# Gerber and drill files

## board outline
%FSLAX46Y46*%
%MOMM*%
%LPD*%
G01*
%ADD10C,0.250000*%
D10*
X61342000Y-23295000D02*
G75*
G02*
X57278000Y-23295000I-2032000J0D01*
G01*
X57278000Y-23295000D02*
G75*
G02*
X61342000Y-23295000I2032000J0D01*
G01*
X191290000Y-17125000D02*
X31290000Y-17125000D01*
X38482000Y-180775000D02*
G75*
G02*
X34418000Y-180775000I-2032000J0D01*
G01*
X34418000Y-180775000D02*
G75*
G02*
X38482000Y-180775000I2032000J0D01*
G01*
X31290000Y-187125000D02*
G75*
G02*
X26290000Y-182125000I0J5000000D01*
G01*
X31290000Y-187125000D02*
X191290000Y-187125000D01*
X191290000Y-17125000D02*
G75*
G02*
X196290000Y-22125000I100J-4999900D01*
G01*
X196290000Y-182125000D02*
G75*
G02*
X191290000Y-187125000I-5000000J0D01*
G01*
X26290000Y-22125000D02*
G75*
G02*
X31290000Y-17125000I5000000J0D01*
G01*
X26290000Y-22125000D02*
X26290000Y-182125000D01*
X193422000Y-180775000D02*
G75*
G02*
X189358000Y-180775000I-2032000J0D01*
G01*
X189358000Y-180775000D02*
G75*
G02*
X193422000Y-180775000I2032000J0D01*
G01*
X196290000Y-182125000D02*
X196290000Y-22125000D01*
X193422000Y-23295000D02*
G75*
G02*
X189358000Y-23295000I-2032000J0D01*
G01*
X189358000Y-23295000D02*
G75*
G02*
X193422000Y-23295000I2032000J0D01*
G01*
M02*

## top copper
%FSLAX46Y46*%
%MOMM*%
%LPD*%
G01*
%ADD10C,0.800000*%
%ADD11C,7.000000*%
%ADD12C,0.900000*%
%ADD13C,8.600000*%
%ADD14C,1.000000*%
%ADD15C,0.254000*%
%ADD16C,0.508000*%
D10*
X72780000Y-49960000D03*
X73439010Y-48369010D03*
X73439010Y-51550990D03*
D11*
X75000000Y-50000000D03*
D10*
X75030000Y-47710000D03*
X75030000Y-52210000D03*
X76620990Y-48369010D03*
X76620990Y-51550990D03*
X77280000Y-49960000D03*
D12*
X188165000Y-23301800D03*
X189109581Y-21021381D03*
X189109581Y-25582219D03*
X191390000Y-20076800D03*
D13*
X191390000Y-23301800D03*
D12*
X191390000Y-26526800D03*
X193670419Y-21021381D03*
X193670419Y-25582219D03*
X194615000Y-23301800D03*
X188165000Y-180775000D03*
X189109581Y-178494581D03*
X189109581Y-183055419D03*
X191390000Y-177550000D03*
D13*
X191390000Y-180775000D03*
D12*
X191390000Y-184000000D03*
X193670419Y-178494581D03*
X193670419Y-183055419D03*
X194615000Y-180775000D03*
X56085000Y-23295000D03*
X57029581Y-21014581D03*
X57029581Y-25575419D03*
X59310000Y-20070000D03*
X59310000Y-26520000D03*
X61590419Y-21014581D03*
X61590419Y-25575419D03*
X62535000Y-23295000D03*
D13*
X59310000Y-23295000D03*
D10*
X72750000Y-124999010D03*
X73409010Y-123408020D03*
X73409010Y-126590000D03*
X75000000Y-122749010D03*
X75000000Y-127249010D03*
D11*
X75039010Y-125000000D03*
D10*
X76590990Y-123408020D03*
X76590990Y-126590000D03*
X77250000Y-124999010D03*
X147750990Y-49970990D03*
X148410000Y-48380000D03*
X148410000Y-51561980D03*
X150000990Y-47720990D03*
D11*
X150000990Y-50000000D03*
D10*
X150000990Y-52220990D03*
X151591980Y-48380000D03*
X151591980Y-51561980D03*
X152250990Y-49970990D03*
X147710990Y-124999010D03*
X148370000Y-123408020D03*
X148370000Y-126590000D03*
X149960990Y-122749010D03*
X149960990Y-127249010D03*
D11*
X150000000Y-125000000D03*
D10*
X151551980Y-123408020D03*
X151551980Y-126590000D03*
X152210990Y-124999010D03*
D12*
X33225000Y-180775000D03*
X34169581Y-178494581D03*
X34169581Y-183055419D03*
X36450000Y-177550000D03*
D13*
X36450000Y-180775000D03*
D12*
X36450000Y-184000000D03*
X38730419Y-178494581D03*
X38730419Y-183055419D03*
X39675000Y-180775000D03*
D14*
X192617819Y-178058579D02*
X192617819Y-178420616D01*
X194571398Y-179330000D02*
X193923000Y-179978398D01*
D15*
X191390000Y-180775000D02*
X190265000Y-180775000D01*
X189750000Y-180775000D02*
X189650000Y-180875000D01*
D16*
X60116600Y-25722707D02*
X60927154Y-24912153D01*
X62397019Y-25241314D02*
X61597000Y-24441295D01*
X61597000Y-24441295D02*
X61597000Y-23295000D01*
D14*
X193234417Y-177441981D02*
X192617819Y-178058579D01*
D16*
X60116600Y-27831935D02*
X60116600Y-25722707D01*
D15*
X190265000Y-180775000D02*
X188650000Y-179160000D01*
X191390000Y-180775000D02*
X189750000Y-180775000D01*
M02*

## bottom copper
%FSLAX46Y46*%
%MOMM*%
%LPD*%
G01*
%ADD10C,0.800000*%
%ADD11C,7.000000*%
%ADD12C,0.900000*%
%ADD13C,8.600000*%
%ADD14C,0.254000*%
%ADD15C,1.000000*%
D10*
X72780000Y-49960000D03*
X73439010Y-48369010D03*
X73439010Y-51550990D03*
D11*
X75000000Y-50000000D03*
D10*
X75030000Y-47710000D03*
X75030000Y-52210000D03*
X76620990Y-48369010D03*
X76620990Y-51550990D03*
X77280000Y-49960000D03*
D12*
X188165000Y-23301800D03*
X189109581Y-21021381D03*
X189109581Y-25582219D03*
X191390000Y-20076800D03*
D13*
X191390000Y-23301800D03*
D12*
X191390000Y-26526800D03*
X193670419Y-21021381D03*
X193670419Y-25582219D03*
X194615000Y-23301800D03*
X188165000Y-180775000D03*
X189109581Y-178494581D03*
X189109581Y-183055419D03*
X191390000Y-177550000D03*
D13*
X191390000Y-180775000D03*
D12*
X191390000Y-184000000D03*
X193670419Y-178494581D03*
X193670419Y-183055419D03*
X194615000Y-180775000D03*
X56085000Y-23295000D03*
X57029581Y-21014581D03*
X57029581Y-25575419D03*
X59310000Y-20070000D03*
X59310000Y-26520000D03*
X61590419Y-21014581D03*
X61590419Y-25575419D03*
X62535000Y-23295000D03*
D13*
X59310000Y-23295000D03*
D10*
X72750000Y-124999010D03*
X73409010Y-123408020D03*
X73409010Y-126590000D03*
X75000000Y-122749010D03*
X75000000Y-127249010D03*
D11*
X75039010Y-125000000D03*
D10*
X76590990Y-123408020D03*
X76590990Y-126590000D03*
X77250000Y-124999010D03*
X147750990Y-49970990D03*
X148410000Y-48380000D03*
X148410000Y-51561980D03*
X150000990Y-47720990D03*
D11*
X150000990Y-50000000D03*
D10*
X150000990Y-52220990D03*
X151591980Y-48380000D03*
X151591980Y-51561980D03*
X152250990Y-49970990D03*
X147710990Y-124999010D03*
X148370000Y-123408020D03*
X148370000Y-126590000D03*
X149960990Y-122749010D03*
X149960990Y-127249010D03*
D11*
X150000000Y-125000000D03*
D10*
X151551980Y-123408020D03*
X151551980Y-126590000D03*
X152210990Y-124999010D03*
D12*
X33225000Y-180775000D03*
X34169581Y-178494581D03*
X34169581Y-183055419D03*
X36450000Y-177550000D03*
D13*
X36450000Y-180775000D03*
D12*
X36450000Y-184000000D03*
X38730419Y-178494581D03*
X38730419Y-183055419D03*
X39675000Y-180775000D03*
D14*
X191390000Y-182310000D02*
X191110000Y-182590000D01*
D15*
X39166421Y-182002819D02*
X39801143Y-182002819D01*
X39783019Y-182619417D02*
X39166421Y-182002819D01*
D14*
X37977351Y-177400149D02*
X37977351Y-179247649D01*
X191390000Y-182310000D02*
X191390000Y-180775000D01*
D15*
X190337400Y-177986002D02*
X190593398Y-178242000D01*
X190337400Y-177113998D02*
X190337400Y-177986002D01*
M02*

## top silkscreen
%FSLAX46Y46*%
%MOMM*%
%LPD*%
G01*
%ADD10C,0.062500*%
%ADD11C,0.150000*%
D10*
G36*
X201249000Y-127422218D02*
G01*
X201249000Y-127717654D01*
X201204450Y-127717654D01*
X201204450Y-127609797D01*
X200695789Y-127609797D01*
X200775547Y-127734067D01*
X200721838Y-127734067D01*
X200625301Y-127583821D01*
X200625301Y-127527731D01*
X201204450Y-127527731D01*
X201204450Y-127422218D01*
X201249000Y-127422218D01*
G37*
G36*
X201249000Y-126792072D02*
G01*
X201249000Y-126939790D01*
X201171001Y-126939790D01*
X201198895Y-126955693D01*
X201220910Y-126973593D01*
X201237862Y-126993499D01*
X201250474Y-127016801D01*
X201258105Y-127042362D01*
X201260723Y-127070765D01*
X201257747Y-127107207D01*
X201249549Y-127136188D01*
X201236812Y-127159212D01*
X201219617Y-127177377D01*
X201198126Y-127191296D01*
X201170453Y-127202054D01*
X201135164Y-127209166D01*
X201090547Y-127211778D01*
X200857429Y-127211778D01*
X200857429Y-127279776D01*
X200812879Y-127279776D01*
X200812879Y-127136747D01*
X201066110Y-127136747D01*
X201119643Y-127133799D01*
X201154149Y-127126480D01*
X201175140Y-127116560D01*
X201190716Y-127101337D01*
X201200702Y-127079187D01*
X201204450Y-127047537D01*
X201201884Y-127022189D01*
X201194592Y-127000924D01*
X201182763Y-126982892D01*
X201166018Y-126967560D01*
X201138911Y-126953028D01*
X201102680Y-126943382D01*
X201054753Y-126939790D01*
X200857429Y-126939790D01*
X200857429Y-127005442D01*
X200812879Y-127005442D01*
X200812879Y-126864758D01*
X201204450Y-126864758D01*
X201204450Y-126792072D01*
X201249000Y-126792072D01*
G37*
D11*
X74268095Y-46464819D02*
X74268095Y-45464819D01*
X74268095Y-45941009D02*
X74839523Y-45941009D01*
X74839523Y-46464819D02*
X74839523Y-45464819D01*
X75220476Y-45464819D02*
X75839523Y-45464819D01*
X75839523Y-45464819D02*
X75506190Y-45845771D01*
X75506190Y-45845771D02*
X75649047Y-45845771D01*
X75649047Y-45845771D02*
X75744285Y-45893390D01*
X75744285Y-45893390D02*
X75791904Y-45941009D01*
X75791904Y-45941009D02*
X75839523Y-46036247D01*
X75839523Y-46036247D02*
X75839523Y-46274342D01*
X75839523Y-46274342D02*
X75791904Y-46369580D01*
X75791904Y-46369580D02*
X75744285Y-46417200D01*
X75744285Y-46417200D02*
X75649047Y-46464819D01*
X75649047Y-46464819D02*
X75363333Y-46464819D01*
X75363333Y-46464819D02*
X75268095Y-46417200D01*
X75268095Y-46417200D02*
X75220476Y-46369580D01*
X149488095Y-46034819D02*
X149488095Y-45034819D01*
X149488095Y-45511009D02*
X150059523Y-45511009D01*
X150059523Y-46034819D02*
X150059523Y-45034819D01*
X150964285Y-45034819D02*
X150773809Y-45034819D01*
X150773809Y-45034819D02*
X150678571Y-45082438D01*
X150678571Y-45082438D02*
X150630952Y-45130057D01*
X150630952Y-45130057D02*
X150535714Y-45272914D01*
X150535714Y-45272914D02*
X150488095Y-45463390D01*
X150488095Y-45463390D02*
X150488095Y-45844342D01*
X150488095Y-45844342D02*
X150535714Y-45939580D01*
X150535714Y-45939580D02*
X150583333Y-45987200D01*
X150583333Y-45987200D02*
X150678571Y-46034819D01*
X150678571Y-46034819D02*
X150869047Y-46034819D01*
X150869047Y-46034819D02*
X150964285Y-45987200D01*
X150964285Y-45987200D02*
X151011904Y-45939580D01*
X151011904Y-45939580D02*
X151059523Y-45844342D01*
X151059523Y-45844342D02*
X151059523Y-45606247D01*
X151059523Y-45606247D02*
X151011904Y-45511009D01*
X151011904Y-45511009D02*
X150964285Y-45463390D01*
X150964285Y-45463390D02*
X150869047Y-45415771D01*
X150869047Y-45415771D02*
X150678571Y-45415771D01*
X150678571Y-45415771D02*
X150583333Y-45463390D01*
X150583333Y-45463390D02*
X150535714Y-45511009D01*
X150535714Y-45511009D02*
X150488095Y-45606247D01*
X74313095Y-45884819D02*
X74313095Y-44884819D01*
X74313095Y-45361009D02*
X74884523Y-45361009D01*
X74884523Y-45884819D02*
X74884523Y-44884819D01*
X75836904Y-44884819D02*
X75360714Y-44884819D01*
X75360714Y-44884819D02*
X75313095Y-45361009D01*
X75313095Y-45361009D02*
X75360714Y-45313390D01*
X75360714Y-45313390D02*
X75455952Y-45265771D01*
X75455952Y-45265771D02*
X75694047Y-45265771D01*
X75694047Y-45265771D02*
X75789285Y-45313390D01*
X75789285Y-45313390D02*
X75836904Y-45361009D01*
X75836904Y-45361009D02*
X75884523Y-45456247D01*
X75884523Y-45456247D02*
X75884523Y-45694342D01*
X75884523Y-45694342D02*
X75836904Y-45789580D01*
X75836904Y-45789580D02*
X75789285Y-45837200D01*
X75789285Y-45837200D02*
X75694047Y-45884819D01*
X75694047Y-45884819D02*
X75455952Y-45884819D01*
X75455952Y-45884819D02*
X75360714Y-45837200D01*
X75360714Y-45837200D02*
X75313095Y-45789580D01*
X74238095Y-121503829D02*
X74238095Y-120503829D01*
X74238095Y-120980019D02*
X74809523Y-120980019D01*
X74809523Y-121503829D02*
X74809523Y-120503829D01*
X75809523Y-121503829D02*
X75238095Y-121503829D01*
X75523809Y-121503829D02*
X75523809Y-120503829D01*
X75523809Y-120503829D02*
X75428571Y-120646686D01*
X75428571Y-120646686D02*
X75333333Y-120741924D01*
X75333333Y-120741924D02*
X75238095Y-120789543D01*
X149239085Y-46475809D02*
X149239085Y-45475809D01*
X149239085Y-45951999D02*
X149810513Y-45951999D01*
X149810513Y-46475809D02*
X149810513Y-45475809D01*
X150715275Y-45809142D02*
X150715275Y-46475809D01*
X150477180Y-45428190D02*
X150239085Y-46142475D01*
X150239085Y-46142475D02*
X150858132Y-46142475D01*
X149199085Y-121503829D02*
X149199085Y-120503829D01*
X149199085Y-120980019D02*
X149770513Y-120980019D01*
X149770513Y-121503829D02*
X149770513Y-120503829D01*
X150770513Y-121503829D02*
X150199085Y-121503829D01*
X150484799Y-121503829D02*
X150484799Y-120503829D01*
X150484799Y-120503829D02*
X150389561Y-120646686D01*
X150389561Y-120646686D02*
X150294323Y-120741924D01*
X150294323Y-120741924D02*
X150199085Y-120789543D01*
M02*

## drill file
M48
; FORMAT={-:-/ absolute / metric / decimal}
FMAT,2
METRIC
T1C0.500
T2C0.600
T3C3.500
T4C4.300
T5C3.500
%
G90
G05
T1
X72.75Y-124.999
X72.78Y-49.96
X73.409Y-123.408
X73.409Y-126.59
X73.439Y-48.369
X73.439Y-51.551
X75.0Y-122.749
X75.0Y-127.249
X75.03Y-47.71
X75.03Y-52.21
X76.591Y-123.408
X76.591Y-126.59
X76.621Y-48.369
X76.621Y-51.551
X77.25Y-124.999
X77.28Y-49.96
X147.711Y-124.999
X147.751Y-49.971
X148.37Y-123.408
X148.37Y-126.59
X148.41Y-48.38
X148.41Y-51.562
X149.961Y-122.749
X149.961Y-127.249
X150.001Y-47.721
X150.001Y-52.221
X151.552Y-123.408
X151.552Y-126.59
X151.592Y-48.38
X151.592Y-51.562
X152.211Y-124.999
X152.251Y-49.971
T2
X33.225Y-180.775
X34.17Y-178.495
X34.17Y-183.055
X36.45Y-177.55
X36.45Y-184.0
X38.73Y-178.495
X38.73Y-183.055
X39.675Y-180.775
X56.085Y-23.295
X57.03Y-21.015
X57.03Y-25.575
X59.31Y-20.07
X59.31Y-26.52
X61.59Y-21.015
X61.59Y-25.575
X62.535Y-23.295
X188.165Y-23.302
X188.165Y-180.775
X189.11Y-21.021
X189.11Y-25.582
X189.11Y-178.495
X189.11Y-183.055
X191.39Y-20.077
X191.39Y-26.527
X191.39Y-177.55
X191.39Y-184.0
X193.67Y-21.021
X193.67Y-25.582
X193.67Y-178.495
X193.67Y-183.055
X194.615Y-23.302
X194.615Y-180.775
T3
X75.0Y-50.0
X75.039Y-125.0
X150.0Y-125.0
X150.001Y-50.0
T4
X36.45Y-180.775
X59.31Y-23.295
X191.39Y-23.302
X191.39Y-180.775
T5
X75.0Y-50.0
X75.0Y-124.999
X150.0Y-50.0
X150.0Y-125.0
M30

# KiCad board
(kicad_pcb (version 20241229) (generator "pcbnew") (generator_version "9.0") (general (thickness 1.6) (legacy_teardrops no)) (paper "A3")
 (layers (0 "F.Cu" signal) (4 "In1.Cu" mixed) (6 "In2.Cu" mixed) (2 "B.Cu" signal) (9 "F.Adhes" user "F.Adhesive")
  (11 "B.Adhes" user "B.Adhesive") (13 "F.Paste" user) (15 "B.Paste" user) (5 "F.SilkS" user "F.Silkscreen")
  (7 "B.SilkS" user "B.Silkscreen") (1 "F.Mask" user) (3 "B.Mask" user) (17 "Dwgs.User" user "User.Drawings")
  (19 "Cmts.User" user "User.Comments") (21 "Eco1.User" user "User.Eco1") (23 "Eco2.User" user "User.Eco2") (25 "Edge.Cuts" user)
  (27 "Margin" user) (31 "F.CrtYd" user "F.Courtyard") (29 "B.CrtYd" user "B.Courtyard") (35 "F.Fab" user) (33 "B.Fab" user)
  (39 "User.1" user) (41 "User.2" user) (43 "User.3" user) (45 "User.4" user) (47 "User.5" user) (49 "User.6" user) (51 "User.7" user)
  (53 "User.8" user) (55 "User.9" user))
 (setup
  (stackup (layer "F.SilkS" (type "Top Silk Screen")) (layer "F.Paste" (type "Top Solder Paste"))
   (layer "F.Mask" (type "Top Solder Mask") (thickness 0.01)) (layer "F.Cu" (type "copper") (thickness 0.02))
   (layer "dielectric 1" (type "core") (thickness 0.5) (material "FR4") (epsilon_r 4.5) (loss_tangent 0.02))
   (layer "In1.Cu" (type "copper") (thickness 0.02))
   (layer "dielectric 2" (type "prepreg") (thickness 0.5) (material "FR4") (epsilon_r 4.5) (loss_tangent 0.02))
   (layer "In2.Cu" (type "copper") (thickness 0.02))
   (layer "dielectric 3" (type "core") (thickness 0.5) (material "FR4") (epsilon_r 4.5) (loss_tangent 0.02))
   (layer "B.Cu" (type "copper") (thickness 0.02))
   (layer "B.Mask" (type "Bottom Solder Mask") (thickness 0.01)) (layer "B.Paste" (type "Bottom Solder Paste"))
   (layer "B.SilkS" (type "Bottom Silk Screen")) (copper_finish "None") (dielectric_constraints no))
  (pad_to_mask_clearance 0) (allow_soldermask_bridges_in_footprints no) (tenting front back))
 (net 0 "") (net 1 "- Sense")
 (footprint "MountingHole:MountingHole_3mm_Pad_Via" (layer "F.Cu") (at 75.03 49.96)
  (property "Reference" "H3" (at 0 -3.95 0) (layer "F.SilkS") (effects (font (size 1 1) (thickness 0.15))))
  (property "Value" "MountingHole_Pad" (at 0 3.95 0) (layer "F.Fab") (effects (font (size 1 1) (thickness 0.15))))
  (pad "1" thru_hole circle (at -2.25 0) (size 0.8 0.8) (drill 0.5) (layers "*.Cu" "*.Mask") (remove_unused_layers no) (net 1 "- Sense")
   (zone_connect 2))
  (pad "1" thru_hole circle (at -1.59099 -1.59099) (size 0.8 0.8) (drill 0.5) (layers "*.Cu" "*.Mask") (remove_unused_layers no)
   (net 1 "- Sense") (zone_connect 2))
  (pad "1" thru_hole circle (at -1.59099 1.59099) (size 0.8 0.8) (drill 0.5) (layers "*.Cu" "*.Mask") (remove_unused_layers no)
   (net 1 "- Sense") (zone_connect 2))
  (pad "1" thru_hole circle (at -0.03 0.04) (size 7 7) (drill 3.5) (layers "*.Cu" "*.Mask") (remove_unused_layers no) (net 1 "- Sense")
   (zone_connect 2))
  (pad "1" thru_hole circle (at 0 -2.25) (size 0.8 0.8) (drill 0.5) (layers "*.Cu" "*.Mask") (remove_unused_layers no) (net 1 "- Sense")
   (zone_connect 2))
  (pad "1" thru_hole circle (at 0 2.25) (size 0.8 0.8) (drill 0.5) (layers "*.Cu" "*.Mask") (remove_unused_layers no) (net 1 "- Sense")
   (zone_connect 2))
  (pad "1" thru_hole circle (at 1.59099 -1.59099) (size 0.8 0.8) (drill 0.5) (layers "*.Cu" "*.Mask") (remove_unused_layers no)
   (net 1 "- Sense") (zone_connect 2))
  (pad "1" thru_hole circle (at 1.59099 1.59099) (size 0.8 0.8) (drill 0.5) (layers "*.Cu" "*.Mask") (remove_unused_layers no)
   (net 1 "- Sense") (zone_connect 2))
  (pad "1" thru_hole circle (at 2.25 0) (size 0.8 0.8) (drill 0.5) (layers "*.Cu" "*.Mask") (remove_unused_layers no) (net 1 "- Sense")
   (zone_connect 2)))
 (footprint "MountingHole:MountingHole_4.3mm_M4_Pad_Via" (layer "F.Cu") (at 191.39 23.3018)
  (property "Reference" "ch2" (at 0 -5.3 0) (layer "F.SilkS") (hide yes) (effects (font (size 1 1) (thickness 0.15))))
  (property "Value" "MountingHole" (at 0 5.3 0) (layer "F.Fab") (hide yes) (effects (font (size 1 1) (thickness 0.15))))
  (pad "1" thru_hole circle (at -3.225 0) (size 0.9 0.9) (drill 0.6) (layers "*.Cu" "*.Mask") (remove_unused_layers no))
  (pad "1" thru_hole circle (at -2.280419 -2.280419) (size 0.9 0.9) (drill 0.6) (layers "*.Cu" "*.Mask") (remove_unused_layers no))
  (pad "1" thru_hole circle (at -2.280419 2.280419) (size 0.9 0.9) (drill 0.6) (layers "*.Cu" "*.Mask") (remove_unused_layers no))
  (pad "1" thru_hole circle (at 0 -3.225) (size 0.9 0.9) (drill 0.6) (layers "*.Cu" "*.Mask") (remove_unused_layers no))
  (pad "1" thru_hole circle (at 0 0) (size 8.6 8.6) (drill 4.3) (layers "*.Cu" "*.Mask") (remove_unused_layers no) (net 1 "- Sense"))
  (pad "1" thru_hole circle (at 0 3.225) (size 0.9 0.9) (drill 0.6) (layers "*.Cu" "*.Mask") (remove_unused_layers no))
  (pad "1" thru_hole circle (at 2.280419 -2.280419) (size 0.9 0.9) (drill 0.6) (layers "*.Cu" "*.Mask") (remove_unused_layers no))
  (pad "1" thru_hole circle (at 2.280419 2.280419) (size 0.9 0.9) (drill 0.6) (layers "*.Cu" "*.Mask") (remove_unused_layers no))
  (pad "1" thru_hole circle (at 3.225 0) (size 0.9 0.9) (drill 0.6) (layers "*.Cu" "*.Mask") (remove_unused_layers no)))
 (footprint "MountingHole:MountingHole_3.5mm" (layer "F.Cu") (at 150 50)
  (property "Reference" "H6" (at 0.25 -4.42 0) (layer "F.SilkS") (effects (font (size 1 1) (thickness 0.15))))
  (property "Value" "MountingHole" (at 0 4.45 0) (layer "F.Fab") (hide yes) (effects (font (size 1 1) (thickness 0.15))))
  (pad "" np_thru_hole circle (at 0 0) (size 3.5 3.5) (drill 3.5) (layers "*.Cu" "*.Mask")))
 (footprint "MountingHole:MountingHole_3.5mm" (layer "F.Cu") (at 150 125)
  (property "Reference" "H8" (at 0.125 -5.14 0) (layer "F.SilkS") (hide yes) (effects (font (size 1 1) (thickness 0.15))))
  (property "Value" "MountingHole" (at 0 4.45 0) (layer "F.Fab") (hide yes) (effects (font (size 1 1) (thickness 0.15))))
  (pad "" np_thru_hole circle (at 0 0) (size 3.5 3.5) (drill 3.5) (layers "*.Cu" "*.Mask")))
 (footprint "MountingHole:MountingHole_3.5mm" (layer "F.Cu") (at 75 50)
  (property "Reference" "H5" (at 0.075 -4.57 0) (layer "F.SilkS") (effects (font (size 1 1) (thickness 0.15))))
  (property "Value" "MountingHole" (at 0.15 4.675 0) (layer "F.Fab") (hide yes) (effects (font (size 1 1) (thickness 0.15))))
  (pad "" np_thru_hole circle (at 0 0) (size 3.5 3.5) (drill 3.5) (layers "*.Cu" "*.Mask")))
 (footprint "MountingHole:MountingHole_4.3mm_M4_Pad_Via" (layer "F.Cu") (at 191.39 180.775)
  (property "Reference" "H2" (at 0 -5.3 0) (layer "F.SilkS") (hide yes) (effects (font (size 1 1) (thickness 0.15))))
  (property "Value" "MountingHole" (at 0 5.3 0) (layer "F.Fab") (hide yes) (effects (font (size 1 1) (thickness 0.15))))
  (pad "1" thru_hole circle (at -3.225 0) (size 0.9 0.9) (drill 0.6) (layers "*.Cu" "*.Mask") (remove_unused_layers no))
  (pad "1" thru_hole circle (at -2.280419 -2.280419) (size 0.9 0.9) (drill 0.6) (layers "*.Cu" "*.Mask") (remove_unused_layers no))
  (pad "1" thru_hole circle (at -2.280419 2.280419) (size 0.9 0.9) (drill 0.6) (layers "*.Cu" "*.Mask") (remove_unused_layers no))
  (pad "1" thru_hole circle (at 0 -3.225) (size 0.9 0.9) (drill 0.6) (layers "*.Cu" "*.Mask") (remove_unused_layers no))
  (pad "1" thru_hole circle (at 0 0) (size 8.6 8.6) (drill 4.3) (layers "*.Cu" "*.Mask") (remove_unused_layers no) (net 1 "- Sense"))
  (pad "1" thru_hole circle (at 0 3.225) (size 0.9 0.9) (drill 0.6) (layers "*.Cu" "*.Mask") (remove_unused_layers no))
  (pad "1" thru_hole circle (at 2.280419 -2.280419) (size 0.9 0.9) (drill 0.6) (layers "*.Cu" "*.Mask") (remove_unused_layers no))
  (pad "1" thru_hole circle (at 2.280419 2.280419) (size 0.9 0.9) (drill 0.6) (layers "*.Cu" "*.Mask") (remove_unused_layers no))
  (pad "1" thru_hole circle (at 3.225 0) (size 0.9 0.9) (drill 0.6) (layers "*.Cu" "*.Mask") (remove_unused_layers no)))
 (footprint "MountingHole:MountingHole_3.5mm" (layer "F.Cu") (at 75 124.99901)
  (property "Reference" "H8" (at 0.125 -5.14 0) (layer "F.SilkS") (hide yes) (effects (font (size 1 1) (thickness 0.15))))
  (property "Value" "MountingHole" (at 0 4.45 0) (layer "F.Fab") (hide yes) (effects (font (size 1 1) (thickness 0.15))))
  (pad "" np_thru_hole circle (at 0 0) (size 3.5 3.5) (drill 3.5) (layers "*.Cu" "*.Mask")))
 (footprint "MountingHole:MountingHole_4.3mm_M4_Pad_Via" (layer "F.Cu") (at 59.31 23.295)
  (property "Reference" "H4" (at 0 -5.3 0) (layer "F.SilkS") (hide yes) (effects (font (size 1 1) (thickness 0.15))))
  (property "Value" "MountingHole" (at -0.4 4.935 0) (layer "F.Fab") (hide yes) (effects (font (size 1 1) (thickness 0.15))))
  (pad "1" thru_hole circle (at -3.225 0) (size 0.9 0.9) (drill 0.6) (layers "*.Cu" "*.Mask") (remove_unused_layers no))
  (pad "1" thru_hole circle (at -2.280419 -2.280419) (size 0.9 0.9) (drill 0.6) (layers "*.Cu" "*.Mask") (remove_unused_layers no))
  (pad "1" thru_hole circle (at -2.280419 2.280419) (size 0.9 0.9) (drill 0.6) (layers "*.Cu" "*.Mask") (remove_unused_layers no))
  (pad "1" thru_hole circle (at 0 -3.225) (size 0.9 0.9) (drill 0.6) (layers "*.Cu" "*.Mask") (remove_unused_layers no))
  (pad "1" thru_hole circle (at 0 3.225) (size 0.9 0.9) (drill 0.6) (layers "*.Cu" "*.Mask") (remove_unused_layers no))
  (pad "1" thru_hole circle (at 2.280419 -2.280419) (size 0.9 0.9) (drill 0.6) (layers "*.Cu" "*.Mask") (remove_unused_layers no))
  (pad "1" thru_hole circle (at 2.280419 2.280419) (size 0.9 0.9) (drill 0.6) (layers "*.Cu" "*.Mask") (remove_unused_layers no))
  (pad "1" thru_hole circle (at 3.225 0) (size 0.9 0.9) (drill 0.6) (layers "*.Cu" "*.Mask") (remove_unused_layers no))
  (pad "ch1" thru_hole circle (at 0 0) (size 8.6 8.6) (drill 4.3) (layers "*.Cu" "*.Mask") (remove_unused_layers no) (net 1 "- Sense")))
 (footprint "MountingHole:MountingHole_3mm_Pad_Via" (layer "F.Cu") (at 75 124.99901)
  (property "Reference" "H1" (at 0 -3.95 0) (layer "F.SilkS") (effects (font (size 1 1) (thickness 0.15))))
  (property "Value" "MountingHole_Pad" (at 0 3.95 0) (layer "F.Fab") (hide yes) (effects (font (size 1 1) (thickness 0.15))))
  (pad "1" thru_hole circle (at -2.25 0) (size 0.8 0.8) (drill 0.5) (layers "*.Cu" "*.Mask") (remove_unused_layers no) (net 1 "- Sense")
   (zone_connect 2))
  (pad "1" thru_hole circle (at -1.59099 -1.59099) (size 0.8 0.8) (drill 0.5) (layers "*.Cu" "*.Mask") (remove_unused_layers no)
   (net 1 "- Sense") (zone_connect 2))
  (pad "1" thru_hole circle (at -1.59099 1.59099) (size 0.8 0.8) (drill 0.5) (layers "*.Cu" "*.Mask") (remove_unused_layers no)
   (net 1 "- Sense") (zone_connect 2))
  (pad "1" thru_hole circle (at 0 -2.25) (size 0.8 0.8) (drill 0.5) (layers "*.Cu" "*.Mask") (remove_unused_layers no) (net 1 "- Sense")
   (zone_connect 2))
  (pad "1" thru_hole circle (at 0 2.25) (size 0.8 0.8) (drill 0.5) (layers "*.Cu" "*.Mask") (remove_unused_layers no) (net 1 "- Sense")
   (zone_connect 2))
  (pad "1" thru_hole circle (at 0.03901 0.00099) (size 7 7) (drill 3.5) (layers "*.Cu" "*.Mask") (remove_unused_layers no) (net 1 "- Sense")
   (zone_connect 2))
  (pad "1" thru_hole circle (at 1.59099 -1.59099) (size 0.8 0.8) (drill 0.5) (layers "*.Cu" "*.Mask") (remove_unused_layers no)
   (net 1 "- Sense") (zone_connect 2))
  (pad "1" thru_hole circle (at 1.59099 1.59099) (size 0.8 0.8) (drill 0.5) (layers "*.Cu" "*.Mask") (remove_unused_layers no)
   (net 1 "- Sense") (zone_connect 2))
  (pad "1" thru_hole circle (at 2.25 0) (size 0.8 0.8) (drill 0.5) (layers "*.Cu" "*.Mask") (remove_unused_layers no) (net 1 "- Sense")
   (zone_connect 2)))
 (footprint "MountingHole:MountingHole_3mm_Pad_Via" (layer "F.Cu") (at 150.00099 49.97099)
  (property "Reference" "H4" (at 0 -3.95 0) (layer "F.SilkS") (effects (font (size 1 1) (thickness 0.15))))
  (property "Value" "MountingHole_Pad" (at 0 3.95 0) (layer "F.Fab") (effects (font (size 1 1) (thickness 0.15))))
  (pad "1" thru_hole circle (at -2.25 0) (size 0.8 0.8) (drill 0.5) (layers "*.Cu" "*.Mask") (remove_unused_layers no) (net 1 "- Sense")
   (zone_connect 2))
  (pad "1" thru_hole circle (at -1.59099 -1.59099) (size 0.8 0.8) (drill 0.5) (layers "*.Cu" "*.Mask") (remove_unused_layers no)
   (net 1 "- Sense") (zone_connect 2))
  (pad "1" thru_hole circle (at -1.59099 1.59099) (size 0.8 0.8) (drill 0.5) (layers "*.Cu" "*.Mask") (remove_unused_layers no)
   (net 1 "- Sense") (zone_connect 2))
  (pad "1" thru_hole circle (at 0 -2.25) (size 0.8 0.8) (drill 0.5) (layers "*.Cu" "*.Mask") (remove_unused_layers no) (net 1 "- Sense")
   (zone_connect 2))
  (pad "1" thru_hole circle (at 0 0.02901) (size 7 7) (drill 3.5) (layers "*.Cu" "*.Mask") (remove_unused_layers no) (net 1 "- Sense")
   (zone_connect 2))
  (pad "1" thru_hole circle (at 0 2.25) (size 0.8 0.8) (drill 0.5) (layers "*.Cu" "*.Mask") (remove_unused_layers no) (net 1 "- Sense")
   (zone_connect 2))
  (pad "1" thru_hole circle (at 1.59099 -1.59099) (size 0.8 0.8) (drill 0.5) (layers "*.Cu" "*.Mask") (remove_unused_layers no)
   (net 1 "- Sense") (zone_connect 2))
  (pad "1" thru_hole circle (at 1.59099 1.59099) (size 0.8 0.8) (drill 0.5) (layers "*.Cu" "*.Mask") (remove_unused_layers no)
   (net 1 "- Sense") (zone_connect 2))
  (pad "1" thru_hole circle (at 2.25 0) (size 0.8 0.8) (drill 0.5) (layers "*.Cu" "*.Mask") (remove_unused_layers no) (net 1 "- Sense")
   (zone_connect 2)))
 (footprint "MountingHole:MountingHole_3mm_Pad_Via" (layer "F.Cu") (at 149.96099 124.99901)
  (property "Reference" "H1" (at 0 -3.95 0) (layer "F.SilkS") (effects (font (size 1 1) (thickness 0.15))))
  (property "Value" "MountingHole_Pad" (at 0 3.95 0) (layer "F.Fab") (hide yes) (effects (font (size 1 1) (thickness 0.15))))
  (pad "1" thru_hole circle (at -2.25 0) (size 0.8 0.8) (drill 0.5) (layers "*.Cu" "*.Mask") (remove_unused_layers no) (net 1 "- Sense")
   (zone_connect 2))
  (pad "1" thru_hole circle (at -1.59099 -1.59099) (size 0.8 0.8) (drill 0.5) (layers "*.Cu" "*.Mask") (remove_unused_layers no)
   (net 1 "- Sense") (zone_connect 2))
  (pad "1" thru_hole circle (at -1.59099 1.59099) (size 0.8 0.8) (drill 0.5) (layers "*.Cu" "*.Mask") (remove_unused_layers no)
   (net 1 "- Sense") (zone_connect 2))
  (pad "1" thru_hole circle (at 0 -2.25) (size 0.8 0.8) (drill 0.5) (layers "*.Cu" "*.Mask") (remove_unused_layers no) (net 1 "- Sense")
   (zone_connect 2))
  (pad "1" thru_hole circle (at 0 2.25) (size 0.8 0.8) (drill 0.5) (layers "*.Cu" "*.Mask") (remove_unused_layers no) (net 1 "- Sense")
   (zone_connect 2))
  (pad "1" thru_hole circle (at 0.03901 0.00099) (size 7 7) (drill 3.5) (layers "*.Cu" "*.Mask") (remove_unused_layers no) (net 1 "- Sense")
   (zone_connect 2))
  (pad "1" thru_hole circle (at 1.59099 -1.59099) (size 0.8 0.8) (drill 0.5) (layers "*.Cu" "*.Mask") (remove_unused_layers no)
   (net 1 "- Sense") (zone_connect 2))
  (pad "1" thru_hole circle (at 1.59099 1.59099) (size 0.8 0.8) (drill 0.5) (layers "*.Cu" "*.Mask") (remove_unused_layers no)
   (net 1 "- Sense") (zone_connect 2))
  (pad "1" thru_hole circle (at 2.25 0) (size 0.8 0.8) (drill 0.5) (layers "*.Cu" "*.Mask") (remove_unused_layers no) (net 1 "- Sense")
   (zone_connect 2)))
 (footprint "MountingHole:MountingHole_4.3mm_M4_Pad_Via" (layer "F.Cu") (at 36.45 180.775)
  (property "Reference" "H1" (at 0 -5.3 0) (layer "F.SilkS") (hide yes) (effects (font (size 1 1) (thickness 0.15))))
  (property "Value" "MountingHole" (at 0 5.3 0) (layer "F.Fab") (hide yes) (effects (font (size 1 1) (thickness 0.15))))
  (pad "1" thru_hole circle (at -3.225 0) (size 0.9 0.9) (drill 0.6) (layers "*.Cu" "*.Mask") (remove_unused_layers no))
  (pad "1" thru_hole circle (at -2.280419 -2.280419) (size 0.9 0.9) (drill 0.6) (layers "*.Cu" "*.Mask") (remove_unused_layers no))
  (pad "1" thru_hole circle (at -2.280419 2.280419) (size 0.9 0.9) (drill 0.6) (layers "*.Cu" "*.Mask") (remove_unused_layers no))
  (pad "1" thru_hole circle (at 0 -3.225) (size 0.9 0.9) (drill 0.6) (layers "*.Cu" "*.Mask") (remove_unused_layers no))
  (pad "1" thru_hole circle (at 0 0) (size 8.6 8.6) (drill 4.3) (layers "*.Cu" "*.Mask") (remove_unused_layers no) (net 1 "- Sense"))
  (pad "1" thru_hole circle (at 0 3.225) (size 0.9 0.9) (drill 0.6) (layers "*.Cu" "*.Mask") (remove_unused_layers no))
  (pad "1" thru_hole circle (at 2.280419 -2.280419) (size 0.9 0.9) (drill 0.6) (layers "*.Cu" "*.Mask") (remove_unused_layers no))
  (pad "1" thru_hole circle (at 2.280419 2.280419) (size 0.9 0.9) (drill 0.6) (layers "*.Cu" "*.Mask") (remove_unused_layers no))
  (pad "1" thru_hole circle (at 3.225 0) (size 0.9 0.9) (drill 0.6) (layers "*.Cu" "*.Mask") (remove_unused_layers no)))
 (gr_circle (center 59.31 23.295) (end 61.342 23.295) (stroke (width 0.25) (type solid)) (fill no) (layer "Edge.Cuts"))
 (gr_line (start 191.29 17.125) (end 31.29 17.125) (stroke (width 0.25) (type solid)) (layer "Edge.Cuts"))
 (gr_circle (center 36.45 180.775) (end 38.482 180.775) (stroke (width 0.25) (type solid)) (fill no) (layer "Edge.Cuts"))
 (gr_arc (start 31.29 187.125) (mid 27.754466 185.660534) (end 26.29 182.125) (stroke (width 0.25) (type solid)) (layer "Edge.Cuts"))
 (gr_line (start 31.29 187.125) (end 191.29 187.125) (stroke (width 0.25) (type solid)) (layer "Edge.Cuts"))
 (gr_arc (start 191.29 17.125) (mid 194.825563 18.589437) (end 196.29 22.125) (stroke (width 0.25) (type solid)) (layer "Edge.Cuts"))
 (gr_arc (start 196.29 182.125) (mid 194.825534 185.660534) (end 191.29 187.125) (stroke (width 0.25) (type solid)) (layer "Edge.Cuts"))
 (gr_arc (start 26.29 22.125) (mid 27.754466 18.589466) (end 31.29 17.125) (stroke (width 0.25) (type solid)) (layer "Edge.Cuts"))
 (gr_line (start 26.29 22.125) (end 26.29 182.125) (stroke (width 0.25) (type solid)) (layer "Edge.Cuts"))
 (gr_circle (center 191.39 180.775) (end 193.422 180.775) (stroke (width 0.25) (type solid)) (fill no) (layer "Edge.Cuts"))
 (gr_line (start 196.29 182.125) (end 196.29 22.125) (stroke (width 0.25) (type solid)) (layer "Edge.Cuts"))
 (gr_circle (center 191.39 23.295) (end 193.422 23.295) (stroke (width 0.25) (type solid)) (fill no) (layer "Edge.Cuts"))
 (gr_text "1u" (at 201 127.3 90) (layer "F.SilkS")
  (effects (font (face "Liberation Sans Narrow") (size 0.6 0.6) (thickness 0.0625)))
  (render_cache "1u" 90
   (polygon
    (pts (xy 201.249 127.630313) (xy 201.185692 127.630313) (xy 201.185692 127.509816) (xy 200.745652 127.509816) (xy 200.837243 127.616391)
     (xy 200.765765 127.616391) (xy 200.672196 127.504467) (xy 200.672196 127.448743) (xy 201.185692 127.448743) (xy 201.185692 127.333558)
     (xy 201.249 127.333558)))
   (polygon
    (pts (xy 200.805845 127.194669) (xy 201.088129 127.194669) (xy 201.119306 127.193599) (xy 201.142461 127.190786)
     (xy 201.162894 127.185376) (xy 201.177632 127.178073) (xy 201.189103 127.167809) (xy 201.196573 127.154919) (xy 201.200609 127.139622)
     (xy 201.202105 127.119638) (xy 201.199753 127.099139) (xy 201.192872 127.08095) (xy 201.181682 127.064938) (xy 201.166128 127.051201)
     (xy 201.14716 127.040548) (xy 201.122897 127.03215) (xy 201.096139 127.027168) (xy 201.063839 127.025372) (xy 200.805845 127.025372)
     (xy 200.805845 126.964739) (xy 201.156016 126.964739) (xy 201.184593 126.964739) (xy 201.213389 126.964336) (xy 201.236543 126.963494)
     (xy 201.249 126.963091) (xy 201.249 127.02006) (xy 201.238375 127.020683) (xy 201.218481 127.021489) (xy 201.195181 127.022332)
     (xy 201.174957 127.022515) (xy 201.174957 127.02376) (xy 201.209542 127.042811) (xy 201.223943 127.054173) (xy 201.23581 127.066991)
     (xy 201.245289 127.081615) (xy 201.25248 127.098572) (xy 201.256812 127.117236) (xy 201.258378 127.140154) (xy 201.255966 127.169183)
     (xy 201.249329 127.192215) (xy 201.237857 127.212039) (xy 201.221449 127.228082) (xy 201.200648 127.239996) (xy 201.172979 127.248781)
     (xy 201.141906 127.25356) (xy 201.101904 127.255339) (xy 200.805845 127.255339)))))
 (segment (start 192.617819 178.058579) (end 192.617819 178.420616) (width 1) (layer "F.Cu") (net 1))
 (segment (start 194.571398 179.33) (end 193.923 179.978398) (width 1) (layer "F.Cu") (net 1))
 (segment (start 191.39 180.775) (end 190.265 180.775) (width 0.254) (layer "F.Cu") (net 1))
 (segment (start 189.75 180.775) (end 189.65 180.875) (width 0.254) (layer "F.Cu") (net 1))
 (segment (start 60.1166 25.722707) (end 60.927154 24.912153) (width 0.508) (layer "F.Cu") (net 1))
 (segment (start 62.397019 25.241314) (end 61.597 24.441295) (width 0.508) (layer "F.Cu") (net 1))
 (segment (start 61.597 24.441295) (end 61.597 23.295) (width 0.508) (layer "F.Cu") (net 1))
 (segment (start 193.234417 177.441981) (end 192.617819 178.058579) (width 1) (layer "F.Cu") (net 1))
 (segment (start 60.1166 27.831935) (end 60.1166 25.722707) (width 0.508) (layer "F.Cu") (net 1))
 (segment (start 190.265 180.775) (end 188.65 179.16) (width 0.254) (layer "F.Cu") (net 1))
 (segment (start 191.39 180.775) (end 189.75 180.775) (width 0.254) (layer "F.Cu") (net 1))
 (segment (start 191.39 182.31) (end 191.11 182.59) (width 0.254) (layer "B.Cu") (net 1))
 (segment (start 39.166421 182.002819) (end 39.801143 182.002819) (width 1) (layer "B.Cu") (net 1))
 (segment (start 39.783019 182.619417) (end 39.166421 182.002819) (width 1) (layer "B.Cu") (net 1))
 (segment (start 37.977351 177.400149) (end 37.977351 179.247649) (width 0.254) (layer "B.Cu") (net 1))
 (segment (start 191.39 182.31) (end 191.39 180.775) (width 0.254) (layer "B.Cu") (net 1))
 (segment (start 190.3374 177.986002) (end 190.593398 178.242) (width 1) (layer "B.Cu") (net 1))
 (segment (start 190.3374 177.113998) (end 190.3374 177.986002) (width 1) (layer "B.Cu") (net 1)))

